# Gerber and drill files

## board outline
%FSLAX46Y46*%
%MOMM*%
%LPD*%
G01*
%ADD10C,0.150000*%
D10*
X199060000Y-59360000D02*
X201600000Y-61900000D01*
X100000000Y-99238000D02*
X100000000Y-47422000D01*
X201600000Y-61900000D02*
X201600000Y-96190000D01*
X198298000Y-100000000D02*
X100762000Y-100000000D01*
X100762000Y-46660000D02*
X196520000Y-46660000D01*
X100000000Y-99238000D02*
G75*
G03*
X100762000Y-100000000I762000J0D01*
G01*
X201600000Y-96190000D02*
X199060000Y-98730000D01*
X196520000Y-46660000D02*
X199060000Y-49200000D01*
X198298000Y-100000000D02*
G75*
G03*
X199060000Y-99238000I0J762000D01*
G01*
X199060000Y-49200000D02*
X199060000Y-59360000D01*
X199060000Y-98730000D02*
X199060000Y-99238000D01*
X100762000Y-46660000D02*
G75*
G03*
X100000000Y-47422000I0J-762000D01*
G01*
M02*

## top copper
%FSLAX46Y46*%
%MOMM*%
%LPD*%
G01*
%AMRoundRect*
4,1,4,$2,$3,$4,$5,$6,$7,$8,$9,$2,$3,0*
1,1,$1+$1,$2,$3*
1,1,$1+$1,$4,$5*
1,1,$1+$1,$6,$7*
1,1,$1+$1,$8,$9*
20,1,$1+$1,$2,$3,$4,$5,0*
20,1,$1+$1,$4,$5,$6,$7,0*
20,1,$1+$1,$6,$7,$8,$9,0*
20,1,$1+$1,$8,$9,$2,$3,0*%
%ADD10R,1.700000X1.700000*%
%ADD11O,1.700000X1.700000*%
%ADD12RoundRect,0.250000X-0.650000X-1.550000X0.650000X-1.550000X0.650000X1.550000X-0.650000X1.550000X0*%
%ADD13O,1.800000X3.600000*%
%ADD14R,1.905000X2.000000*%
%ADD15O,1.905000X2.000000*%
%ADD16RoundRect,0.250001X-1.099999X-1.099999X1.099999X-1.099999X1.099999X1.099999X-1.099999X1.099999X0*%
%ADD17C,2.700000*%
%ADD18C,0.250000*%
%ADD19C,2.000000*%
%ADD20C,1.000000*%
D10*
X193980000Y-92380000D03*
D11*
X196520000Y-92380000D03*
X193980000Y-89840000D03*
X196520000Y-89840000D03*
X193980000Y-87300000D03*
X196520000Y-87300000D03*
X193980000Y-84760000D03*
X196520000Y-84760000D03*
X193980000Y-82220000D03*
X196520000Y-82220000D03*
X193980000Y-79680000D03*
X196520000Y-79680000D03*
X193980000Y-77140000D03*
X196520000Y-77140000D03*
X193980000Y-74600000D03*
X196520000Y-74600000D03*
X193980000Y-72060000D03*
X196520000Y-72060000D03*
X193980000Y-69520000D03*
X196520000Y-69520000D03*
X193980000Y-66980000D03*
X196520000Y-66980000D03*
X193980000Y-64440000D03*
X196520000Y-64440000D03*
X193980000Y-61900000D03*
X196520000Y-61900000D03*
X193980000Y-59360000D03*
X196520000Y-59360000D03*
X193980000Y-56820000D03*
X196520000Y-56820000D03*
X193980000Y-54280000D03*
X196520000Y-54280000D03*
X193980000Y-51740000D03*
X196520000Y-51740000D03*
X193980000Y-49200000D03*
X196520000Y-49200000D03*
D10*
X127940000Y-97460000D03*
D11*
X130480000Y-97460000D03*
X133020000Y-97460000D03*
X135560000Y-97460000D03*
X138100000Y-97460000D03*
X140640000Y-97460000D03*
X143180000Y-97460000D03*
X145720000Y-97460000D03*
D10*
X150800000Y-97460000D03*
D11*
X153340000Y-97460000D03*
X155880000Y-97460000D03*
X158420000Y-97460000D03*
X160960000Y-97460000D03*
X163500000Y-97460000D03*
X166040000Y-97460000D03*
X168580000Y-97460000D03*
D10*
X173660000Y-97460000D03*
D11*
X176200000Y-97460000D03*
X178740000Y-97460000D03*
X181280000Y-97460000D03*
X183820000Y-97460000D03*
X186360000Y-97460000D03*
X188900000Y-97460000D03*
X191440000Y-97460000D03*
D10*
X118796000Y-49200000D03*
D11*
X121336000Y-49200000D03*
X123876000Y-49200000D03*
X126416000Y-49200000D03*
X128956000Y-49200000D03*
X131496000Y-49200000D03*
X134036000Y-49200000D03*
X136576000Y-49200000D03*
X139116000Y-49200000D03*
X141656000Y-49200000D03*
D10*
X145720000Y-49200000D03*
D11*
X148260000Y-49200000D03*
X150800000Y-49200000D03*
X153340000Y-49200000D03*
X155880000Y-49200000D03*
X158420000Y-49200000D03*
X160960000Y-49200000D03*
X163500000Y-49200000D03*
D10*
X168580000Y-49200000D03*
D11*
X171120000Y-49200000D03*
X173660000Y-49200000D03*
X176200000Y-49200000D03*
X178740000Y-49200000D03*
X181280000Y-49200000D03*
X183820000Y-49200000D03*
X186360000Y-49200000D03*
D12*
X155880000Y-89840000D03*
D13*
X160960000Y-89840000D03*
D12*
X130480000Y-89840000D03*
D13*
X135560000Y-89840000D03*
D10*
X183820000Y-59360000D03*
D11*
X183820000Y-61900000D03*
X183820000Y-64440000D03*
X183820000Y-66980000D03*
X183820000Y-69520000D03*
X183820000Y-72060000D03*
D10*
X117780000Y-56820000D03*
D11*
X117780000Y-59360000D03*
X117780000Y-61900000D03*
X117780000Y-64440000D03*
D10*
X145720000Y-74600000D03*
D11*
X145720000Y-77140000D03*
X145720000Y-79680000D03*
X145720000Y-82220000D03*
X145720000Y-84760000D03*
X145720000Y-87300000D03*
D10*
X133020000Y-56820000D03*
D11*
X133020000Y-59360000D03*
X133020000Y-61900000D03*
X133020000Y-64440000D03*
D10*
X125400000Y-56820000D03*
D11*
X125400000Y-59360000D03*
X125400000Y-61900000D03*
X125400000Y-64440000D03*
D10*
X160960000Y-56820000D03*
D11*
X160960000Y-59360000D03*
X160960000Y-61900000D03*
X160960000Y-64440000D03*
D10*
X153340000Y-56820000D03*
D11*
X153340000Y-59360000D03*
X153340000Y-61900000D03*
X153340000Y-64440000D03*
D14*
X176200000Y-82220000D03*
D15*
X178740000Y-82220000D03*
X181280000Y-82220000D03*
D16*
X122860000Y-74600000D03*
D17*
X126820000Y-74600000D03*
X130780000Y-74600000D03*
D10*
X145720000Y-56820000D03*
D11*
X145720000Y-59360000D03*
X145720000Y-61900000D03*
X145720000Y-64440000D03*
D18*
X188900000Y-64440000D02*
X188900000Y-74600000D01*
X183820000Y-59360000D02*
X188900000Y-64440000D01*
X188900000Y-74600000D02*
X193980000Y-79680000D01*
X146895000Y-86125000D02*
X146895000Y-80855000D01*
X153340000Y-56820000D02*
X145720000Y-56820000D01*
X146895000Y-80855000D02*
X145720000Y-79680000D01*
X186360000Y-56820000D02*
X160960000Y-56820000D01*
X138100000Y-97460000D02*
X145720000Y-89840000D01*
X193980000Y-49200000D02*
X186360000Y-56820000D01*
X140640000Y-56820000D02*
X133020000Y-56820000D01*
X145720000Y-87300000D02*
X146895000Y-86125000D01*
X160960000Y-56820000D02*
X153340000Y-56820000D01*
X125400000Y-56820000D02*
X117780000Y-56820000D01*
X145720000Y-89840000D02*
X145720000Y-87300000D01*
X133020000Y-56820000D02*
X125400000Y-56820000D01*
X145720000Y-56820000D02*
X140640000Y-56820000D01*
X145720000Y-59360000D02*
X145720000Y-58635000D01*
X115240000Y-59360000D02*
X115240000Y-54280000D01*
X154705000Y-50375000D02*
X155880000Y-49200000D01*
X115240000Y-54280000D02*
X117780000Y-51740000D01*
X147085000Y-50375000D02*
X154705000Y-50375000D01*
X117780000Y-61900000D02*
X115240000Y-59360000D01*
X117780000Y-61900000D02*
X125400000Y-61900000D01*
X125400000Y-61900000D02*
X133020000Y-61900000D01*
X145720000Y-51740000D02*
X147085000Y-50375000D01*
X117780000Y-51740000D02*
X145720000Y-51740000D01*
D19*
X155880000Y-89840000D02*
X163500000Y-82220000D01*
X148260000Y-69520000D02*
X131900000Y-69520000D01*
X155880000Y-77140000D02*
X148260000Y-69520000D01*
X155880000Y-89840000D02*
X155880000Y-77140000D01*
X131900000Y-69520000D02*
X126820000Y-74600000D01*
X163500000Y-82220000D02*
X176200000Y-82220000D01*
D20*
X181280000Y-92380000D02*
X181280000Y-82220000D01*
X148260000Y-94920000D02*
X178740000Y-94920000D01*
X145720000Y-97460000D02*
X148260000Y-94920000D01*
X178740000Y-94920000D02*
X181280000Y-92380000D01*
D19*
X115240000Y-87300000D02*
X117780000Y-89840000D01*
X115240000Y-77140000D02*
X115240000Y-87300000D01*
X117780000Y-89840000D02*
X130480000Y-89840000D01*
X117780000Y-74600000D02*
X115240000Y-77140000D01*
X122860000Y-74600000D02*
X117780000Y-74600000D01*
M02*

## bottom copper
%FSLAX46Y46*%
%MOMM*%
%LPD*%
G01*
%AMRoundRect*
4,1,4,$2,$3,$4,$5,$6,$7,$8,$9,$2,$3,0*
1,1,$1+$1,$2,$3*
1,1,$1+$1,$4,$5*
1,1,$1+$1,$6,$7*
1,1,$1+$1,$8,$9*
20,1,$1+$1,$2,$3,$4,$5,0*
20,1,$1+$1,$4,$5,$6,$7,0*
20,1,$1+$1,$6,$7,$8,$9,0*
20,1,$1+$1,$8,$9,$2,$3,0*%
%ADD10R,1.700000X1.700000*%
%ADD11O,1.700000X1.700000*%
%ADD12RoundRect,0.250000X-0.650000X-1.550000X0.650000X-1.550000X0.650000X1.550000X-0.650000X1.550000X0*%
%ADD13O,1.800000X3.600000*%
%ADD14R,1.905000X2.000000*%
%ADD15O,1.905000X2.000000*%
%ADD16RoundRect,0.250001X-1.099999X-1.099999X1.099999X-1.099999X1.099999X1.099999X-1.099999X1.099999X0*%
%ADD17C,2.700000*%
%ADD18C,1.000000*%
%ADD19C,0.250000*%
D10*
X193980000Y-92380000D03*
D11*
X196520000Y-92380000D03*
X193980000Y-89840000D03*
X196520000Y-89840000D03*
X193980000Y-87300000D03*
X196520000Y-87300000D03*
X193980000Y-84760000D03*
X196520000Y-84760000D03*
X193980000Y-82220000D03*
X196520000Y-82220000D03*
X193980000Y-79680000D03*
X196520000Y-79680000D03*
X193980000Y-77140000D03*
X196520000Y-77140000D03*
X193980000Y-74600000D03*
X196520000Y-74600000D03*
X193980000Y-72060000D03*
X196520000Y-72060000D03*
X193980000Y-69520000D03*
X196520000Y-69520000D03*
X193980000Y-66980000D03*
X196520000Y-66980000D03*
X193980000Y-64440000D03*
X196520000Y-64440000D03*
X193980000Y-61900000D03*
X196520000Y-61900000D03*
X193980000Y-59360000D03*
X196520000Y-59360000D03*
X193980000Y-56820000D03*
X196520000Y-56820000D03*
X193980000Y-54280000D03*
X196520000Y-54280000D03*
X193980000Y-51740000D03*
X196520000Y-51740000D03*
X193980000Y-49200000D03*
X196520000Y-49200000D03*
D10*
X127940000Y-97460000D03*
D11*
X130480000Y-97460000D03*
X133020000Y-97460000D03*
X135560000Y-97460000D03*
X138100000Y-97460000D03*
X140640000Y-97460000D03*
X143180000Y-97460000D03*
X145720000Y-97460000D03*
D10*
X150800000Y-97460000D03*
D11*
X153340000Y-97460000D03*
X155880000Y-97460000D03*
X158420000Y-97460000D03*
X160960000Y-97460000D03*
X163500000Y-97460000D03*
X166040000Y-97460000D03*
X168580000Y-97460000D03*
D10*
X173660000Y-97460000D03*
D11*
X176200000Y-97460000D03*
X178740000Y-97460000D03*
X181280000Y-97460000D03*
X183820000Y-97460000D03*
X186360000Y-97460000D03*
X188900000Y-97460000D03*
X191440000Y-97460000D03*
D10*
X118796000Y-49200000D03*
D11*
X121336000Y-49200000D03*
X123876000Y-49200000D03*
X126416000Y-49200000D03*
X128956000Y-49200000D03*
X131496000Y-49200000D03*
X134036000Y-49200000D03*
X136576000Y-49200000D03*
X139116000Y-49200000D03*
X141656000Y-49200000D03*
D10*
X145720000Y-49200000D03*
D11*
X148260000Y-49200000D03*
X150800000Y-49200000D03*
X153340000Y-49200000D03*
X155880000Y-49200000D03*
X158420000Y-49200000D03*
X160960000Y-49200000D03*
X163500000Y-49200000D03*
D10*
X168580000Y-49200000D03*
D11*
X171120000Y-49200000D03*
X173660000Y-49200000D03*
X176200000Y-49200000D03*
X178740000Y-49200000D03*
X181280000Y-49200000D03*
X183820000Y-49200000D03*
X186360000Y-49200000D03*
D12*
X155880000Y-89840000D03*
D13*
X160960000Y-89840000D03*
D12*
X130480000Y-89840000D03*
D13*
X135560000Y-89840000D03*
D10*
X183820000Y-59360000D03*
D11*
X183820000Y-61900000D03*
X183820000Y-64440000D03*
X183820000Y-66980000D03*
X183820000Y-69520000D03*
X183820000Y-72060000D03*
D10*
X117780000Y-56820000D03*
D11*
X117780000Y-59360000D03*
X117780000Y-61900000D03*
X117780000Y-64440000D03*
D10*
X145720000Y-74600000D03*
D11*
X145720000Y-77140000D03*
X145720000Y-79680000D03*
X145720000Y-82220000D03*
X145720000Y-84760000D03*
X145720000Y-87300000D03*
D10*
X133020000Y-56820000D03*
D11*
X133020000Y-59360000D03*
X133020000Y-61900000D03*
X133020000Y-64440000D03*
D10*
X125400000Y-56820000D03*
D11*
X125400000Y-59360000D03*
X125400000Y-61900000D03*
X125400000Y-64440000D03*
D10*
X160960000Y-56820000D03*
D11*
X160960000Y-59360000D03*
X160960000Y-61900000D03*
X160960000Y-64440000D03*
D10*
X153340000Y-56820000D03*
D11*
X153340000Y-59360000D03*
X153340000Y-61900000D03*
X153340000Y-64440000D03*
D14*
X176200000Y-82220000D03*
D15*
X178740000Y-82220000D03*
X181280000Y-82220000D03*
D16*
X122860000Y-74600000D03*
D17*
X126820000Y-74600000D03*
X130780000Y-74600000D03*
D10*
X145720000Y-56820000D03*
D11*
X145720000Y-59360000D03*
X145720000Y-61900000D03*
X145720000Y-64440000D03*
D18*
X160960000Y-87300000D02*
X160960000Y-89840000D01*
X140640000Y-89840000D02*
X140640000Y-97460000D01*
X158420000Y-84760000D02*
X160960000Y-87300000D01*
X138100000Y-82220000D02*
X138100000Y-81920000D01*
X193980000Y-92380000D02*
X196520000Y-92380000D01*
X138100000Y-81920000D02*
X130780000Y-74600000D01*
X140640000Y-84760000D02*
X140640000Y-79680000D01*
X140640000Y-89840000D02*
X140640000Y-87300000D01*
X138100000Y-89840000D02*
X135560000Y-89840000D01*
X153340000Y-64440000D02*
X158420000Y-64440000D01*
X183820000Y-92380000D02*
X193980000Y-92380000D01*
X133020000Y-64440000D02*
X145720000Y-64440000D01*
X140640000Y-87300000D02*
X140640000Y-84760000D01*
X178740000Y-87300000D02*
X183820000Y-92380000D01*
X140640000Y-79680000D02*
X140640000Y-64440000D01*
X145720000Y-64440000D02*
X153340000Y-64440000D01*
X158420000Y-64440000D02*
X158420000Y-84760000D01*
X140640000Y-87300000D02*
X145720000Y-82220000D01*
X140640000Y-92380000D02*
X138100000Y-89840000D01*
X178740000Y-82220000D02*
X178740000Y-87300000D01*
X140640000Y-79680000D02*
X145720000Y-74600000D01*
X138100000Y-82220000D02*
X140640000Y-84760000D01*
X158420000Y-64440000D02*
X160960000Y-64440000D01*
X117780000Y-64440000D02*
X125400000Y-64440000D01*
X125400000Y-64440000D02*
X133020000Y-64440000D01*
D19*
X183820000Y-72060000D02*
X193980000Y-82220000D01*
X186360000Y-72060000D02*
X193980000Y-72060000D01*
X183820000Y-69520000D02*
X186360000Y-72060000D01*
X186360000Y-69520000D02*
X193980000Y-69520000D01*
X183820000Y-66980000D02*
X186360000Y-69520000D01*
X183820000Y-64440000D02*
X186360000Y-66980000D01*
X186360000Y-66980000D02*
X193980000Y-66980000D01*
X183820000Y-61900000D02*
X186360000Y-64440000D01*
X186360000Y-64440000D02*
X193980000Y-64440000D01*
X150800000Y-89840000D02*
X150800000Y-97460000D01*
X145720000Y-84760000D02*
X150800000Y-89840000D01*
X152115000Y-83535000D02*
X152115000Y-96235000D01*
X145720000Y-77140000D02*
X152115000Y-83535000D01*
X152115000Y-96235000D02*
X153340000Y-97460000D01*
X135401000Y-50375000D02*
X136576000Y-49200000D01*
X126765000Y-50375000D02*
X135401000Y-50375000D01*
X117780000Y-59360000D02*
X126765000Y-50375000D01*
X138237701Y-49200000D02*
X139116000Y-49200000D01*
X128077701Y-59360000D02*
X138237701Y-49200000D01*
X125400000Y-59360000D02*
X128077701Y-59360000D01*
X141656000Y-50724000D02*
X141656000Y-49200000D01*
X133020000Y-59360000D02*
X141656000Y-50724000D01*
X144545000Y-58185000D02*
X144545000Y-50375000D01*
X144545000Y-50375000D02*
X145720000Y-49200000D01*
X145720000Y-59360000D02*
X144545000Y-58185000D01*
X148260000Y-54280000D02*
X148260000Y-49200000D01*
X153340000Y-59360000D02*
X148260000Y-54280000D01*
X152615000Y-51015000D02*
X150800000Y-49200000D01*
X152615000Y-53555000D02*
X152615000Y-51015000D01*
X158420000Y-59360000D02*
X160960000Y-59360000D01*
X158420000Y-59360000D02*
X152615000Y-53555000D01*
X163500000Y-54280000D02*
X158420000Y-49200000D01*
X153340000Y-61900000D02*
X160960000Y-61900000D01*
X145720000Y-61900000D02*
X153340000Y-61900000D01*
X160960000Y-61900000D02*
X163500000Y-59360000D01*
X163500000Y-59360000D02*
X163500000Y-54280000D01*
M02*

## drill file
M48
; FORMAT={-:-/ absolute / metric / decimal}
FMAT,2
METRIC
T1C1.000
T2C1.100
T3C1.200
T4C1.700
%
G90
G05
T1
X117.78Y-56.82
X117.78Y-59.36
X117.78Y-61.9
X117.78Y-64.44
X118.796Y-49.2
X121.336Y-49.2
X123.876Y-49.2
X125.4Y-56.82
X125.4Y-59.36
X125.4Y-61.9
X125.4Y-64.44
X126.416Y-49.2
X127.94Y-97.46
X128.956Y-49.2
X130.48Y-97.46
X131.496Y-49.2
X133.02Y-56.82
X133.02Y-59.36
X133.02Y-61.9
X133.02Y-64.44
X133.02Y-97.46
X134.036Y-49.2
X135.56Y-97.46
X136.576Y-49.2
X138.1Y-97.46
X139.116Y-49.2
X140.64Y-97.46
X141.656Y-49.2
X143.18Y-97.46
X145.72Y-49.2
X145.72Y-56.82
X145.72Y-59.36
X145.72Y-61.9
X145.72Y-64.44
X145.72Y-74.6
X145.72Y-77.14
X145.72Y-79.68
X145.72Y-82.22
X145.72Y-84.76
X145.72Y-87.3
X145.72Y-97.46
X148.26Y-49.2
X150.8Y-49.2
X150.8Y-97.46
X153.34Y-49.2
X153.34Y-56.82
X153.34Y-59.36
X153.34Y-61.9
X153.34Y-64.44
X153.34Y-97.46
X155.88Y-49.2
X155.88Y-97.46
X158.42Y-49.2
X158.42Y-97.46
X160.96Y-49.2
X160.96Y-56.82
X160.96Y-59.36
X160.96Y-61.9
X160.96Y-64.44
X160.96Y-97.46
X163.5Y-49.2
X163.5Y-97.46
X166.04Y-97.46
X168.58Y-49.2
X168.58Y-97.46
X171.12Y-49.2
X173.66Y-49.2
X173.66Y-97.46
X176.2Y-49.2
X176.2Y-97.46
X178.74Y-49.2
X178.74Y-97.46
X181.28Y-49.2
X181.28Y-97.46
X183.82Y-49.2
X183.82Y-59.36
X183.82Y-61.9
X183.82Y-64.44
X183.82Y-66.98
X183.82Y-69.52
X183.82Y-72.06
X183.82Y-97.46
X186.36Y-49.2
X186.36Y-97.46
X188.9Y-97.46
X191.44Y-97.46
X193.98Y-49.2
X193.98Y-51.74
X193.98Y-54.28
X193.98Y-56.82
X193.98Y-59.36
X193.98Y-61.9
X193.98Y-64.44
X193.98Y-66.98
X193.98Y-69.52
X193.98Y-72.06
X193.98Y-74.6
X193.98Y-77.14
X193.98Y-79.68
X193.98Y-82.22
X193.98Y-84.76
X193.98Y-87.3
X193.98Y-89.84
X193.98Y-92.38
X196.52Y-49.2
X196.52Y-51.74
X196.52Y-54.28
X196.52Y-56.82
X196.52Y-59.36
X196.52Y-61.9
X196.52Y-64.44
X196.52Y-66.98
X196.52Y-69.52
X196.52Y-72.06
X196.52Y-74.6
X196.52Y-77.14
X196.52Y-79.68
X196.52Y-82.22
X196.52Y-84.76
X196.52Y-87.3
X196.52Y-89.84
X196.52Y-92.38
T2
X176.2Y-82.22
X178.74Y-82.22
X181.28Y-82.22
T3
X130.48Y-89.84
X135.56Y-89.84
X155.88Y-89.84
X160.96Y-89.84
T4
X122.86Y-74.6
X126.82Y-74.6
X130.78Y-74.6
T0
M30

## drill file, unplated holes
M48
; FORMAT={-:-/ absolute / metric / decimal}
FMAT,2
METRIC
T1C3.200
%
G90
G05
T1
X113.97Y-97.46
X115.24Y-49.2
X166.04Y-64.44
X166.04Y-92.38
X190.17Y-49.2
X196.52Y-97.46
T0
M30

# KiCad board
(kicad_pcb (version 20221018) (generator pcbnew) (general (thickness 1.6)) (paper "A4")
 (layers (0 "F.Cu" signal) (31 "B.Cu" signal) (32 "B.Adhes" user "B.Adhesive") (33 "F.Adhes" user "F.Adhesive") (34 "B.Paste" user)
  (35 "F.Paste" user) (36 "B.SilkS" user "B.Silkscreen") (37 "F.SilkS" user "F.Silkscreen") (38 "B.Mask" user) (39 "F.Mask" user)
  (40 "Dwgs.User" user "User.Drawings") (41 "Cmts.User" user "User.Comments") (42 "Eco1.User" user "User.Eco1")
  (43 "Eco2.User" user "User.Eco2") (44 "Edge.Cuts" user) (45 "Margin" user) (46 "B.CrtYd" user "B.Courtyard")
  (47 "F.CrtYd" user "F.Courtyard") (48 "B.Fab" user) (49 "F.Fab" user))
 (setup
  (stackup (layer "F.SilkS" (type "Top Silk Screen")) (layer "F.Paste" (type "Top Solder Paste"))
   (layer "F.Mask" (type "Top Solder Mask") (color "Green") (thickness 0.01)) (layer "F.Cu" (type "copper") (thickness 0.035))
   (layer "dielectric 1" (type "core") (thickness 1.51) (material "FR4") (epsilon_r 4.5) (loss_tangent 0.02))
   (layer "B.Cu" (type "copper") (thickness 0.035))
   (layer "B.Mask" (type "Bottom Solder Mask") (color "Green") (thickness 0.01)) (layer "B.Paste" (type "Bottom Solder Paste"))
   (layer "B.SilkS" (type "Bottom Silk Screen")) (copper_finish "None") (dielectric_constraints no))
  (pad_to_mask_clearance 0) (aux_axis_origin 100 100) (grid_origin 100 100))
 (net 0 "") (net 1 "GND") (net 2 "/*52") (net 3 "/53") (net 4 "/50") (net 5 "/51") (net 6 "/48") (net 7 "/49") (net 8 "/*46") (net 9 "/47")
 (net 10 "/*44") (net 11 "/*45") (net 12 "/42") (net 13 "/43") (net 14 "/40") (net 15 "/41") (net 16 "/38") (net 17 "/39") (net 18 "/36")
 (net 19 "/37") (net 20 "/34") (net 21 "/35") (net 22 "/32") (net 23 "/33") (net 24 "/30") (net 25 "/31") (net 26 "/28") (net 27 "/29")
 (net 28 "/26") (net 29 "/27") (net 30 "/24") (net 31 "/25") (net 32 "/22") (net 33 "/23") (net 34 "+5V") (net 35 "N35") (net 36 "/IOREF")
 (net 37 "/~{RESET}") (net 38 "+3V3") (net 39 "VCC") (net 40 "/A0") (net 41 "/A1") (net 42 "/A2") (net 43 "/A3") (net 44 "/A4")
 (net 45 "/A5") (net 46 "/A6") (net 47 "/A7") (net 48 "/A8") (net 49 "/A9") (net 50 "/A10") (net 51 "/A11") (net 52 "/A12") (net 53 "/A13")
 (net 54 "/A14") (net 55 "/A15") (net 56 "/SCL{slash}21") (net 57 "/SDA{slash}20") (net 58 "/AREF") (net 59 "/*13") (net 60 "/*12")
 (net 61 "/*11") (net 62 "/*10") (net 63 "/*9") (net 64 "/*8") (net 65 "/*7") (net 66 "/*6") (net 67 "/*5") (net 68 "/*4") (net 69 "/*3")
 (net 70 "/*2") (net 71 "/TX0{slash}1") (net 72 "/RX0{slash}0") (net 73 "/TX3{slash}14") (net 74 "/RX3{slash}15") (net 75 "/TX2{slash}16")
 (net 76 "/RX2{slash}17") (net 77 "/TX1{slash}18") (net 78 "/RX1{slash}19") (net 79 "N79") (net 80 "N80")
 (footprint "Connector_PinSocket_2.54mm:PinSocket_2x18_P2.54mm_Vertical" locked (layer "F.Cu") (at 193.98 92.38 180)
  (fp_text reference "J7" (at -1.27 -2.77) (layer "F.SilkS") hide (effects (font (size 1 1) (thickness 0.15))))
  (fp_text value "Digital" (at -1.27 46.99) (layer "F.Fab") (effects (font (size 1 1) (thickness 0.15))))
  (pad "1" thru_hole rect locked (at 0 0 180) (size 1.7 1.7) (drill 1) (layers "*.Cu" "*.Mask") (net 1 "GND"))
  (pad "2" thru_hole oval locked (at -2.54 0 180) (size 1.7 1.7) (drill 1) (layers "*.Cu" "*.Mask") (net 1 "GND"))
  (pad "3" thru_hole oval locked (at 0 2.54 180) (size 1.7 1.7) (drill 1) (layers "*.Cu" "*.Mask") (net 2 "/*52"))
  (pad "4" thru_hole oval locked (at -2.54 2.54 180) (size 1.7 1.7) (drill 1) (layers "*.Cu" "*.Mask") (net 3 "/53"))
  (pad "5" thru_hole oval locked (at 0 5.08 180) (size 1.7 1.7) (drill 1) (layers "*.Cu" "*.Mask") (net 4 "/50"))
  (pad "6" thru_hole oval locked (at -2.54 5.08 180) (size 1.7 1.7) (drill 1) (layers "*.Cu" "*.Mask") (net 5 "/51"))
  (pad "7" thru_hole oval locked (at 0 7.62 180) (size 1.7 1.7) (drill 1) (layers "*.Cu" "*.Mask") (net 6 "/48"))
  (pad "8" thru_hole oval locked (at -2.54 7.62 180) (size 1.7 1.7) (drill 1) (layers "*.Cu" "*.Mask") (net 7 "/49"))
  (pad "9" thru_hole oval locked (at 0 10.16 180) (size 1.7 1.7) (drill 1) (layers "*.Cu" "*.Mask") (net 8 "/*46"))
  (pad "10" thru_hole oval locked (at -2.54 10.16 180) (size 1.7 1.7) (drill 1) (layers "*.Cu" "*.Mask") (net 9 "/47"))
  (pad "11" thru_hole oval locked (at 0 12.7 180) (size 1.7 1.7) (drill 1) (layers "*.Cu" "*.Mask") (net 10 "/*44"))
  (pad "12" thru_hole oval locked (at -2.54 12.7 180) (size 1.7 1.7) (drill 1) (layers "*.Cu" "*.Mask") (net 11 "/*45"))
  (pad "13" thru_hole oval locked (at 0 15.24 180) (size 1.7 1.7) (drill 1) (layers "*.Cu" "*.Mask") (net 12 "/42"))
  (pad "14" thru_hole oval locked (at -2.54 15.24 180) (size 1.7 1.7) (drill 1) (layers "*.Cu" "*.Mask") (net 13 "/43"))
  (pad "15" thru_hole oval locked (at 0 17.78 180) (size 1.7 1.7) (drill 1) (layers "*.Cu" "*.Mask") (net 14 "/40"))
  (pad "16" thru_hole oval locked (at -2.54 17.78 180) (size 1.7 1.7) (drill 1) (layers "*.Cu" "*.Mask") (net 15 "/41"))
  (pad "17" thru_hole oval locked (at 0 20.32 180) (size 1.7 1.7) (drill 1) (layers "*.Cu" "*.Mask") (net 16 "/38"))
  (pad "18" thru_hole oval locked (at -2.54 20.32 180) (size 1.7 1.7) (drill 1) (layers "*.Cu" "*.Mask") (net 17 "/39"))
  (pad "19" thru_hole oval locked (at 0 22.86 180) (size 1.7 1.7) (drill 1) (layers "*.Cu" "*.Mask") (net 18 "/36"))
  (pad "20" thru_hole oval locked (at -2.54 22.86 180) (size 1.7 1.7) (drill 1) (layers "*.Cu" "*.Mask") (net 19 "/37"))
  (pad "21" thru_hole oval locked (at 0 25.4 180) (size 1.7 1.7) (drill 1) (layers "*.Cu" "*.Mask") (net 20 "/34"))
  (pad "22" thru_hole oval locked (at -2.54 25.4 180) (size 1.7 1.7) (drill 1) (layers "*.Cu" "*.Mask") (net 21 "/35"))
  (pad "23" thru_hole oval locked (at 0 27.94 180) (size 1.7 1.7) (drill 1) (layers "*.Cu" "*.Mask") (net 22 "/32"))
  (pad "24" thru_hole oval locked (at -2.54 27.94 180) (size 1.7 1.7) (drill 1) (layers "*.Cu" "*.Mask") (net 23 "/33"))
  (pad "25" thru_hole oval locked (at 0 30.48 180) (size 1.7 1.7) (drill 1) (layers "*.Cu" "*.Mask") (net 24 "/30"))
  (pad "26" thru_hole oval locked (at -2.54 30.48 180) (size 1.7 1.7) (drill 1) (layers "*.Cu" "*.Mask") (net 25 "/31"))
  (pad "27" thru_hole oval locked (at 0 33.02 180) (size 1.7 1.7) (drill 1) (layers "*.Cu" "*.Mask") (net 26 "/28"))
  (pad "28" thru_hole oval locked (at -2.54 33.02 180) (size 1.7 1.7) (drill 1) (layers "*.Cu" "*.Mask") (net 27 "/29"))
  (pad "29" thru_hole oval locked (at 0 35.56 180) (size 1.7 1.7) (drill 1) (layers "*.Cu" "*.Mask") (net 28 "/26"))
  (pad "30" thru_hole oval locked (at -2.54 35.56 180) (size 1.7 1.7) (drill 1) (layers "*.Cu" "*.Mask") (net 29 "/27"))
  (pad "31" thru_hole oval locked (at 0 38.1 180) (size 1.7 1.7) (drill 1) (layers "*.Cu" "*.Mask") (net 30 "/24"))
  (pad "32" thru_hole oval locked (at -2.54 38.1 180) (size 1.7 1.7) (drill 1) (layers "*.Cu" "*.Mask") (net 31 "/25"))
  (pad "33" thru_hole oval locked (at 0 40.64 180) (size 1.7 1.7) (drill 1) (layers "*.Cu" "*.Mask") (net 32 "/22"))
  (pad "34" thru_hole oval locked (at -2.54 40.64 180) (size 1.7 1.7) (drill 1) (layers "*.Cu" "*.Mask") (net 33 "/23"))
  (pad "35" thru_hole oval locked (at 0 43.18 180) (size 1.7 1.7) (drill 1) (layers "*.Cu" "*.Mask") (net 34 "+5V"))
  (pad "36" thru_hole oval locked (at -2.54 43.18 180) (size 1.7 1.7) (drill 1) (layers "*.Cu" "*.Mask") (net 34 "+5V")))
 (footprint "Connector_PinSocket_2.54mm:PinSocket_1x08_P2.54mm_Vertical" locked (layer "F.Cu") (at 127.94 97.46 90)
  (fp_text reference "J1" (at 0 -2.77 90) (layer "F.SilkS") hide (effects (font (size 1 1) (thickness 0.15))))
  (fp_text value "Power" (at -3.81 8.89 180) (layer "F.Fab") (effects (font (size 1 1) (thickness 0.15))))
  (pad "1" thru_hole rect locked (at 0 0 90) (size 1.7 1.7) (drill 1) (layers "*.Cu" "*.Mask") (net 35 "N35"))
  (pad "2" thru_hole oval locked (at 0 2.54 90) (size 1.7 1.7) (drill 1) (layers "*.Cu" "*.Mask") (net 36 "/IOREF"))
  (pad "3" thru_hole oval locked (at 0 5.08 90) (size 1.7 1.7) (drill 1) (layers "*.Cu" "*.Mask") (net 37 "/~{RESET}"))
  (pad "4" thru_hole oval locked (at 0 7.62 90) (size 1.7 1.7) (drill 1) (layers "*.Cu" "*.Mask") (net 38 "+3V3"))
  (pad "5" thru_hole oval locked (at 0 10.16 90) (size 1.7 1.7) (drill 1) (layers "*.Cu" "*.Mask") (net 34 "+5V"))
  (pad "6" thru_hole oval locked (at 0 12.7 90) (size 1.7 1.7) (drill 1) (layers "*.Cu" "*.Mask") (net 1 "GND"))
  (pad "7" thru_hole oval locked (at 0 15.24 90) (size 1.7 1.7) (drill 1) (layers "*.Cu" "*.Mask") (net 1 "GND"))
  (pad "8" thru_hole oval locked (at 0 17.78 90) (size 1.7 1.7) (drill 1) (layers "*.Cu" "*.Mask") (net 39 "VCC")))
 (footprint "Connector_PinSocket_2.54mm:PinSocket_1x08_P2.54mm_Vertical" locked (layer "F.Cu") (at 150.8 97.46 90)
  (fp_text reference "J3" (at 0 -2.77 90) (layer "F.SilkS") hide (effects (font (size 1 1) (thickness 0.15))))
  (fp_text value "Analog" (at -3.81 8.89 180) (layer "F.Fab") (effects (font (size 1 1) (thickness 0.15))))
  (pad "1" thru_hole rect locked (at 0 0 90) (size 1.7 1.7) (drill 1) (layers "*.Cu" "*.Mask") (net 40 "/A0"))
  (pad "2" thru_hole oval locked (at 0 2.54 90) (size 1.7 1.7) (drill 1) (layers "*.Cu" "*.Mask") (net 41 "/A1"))
  (pad "3" thru_hole oval locked (at 0 5.08 90) (size 1.7 1.7) (drill 1) (layers "*.Cu" "*.Mask") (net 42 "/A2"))
  (pad "4" thru_hole oval locked (at 0 7.62 90) (size 1.7 1.7) (drill 1) (layers "*.Cu" "*.Mask") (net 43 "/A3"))
  (pad "5" thru_hole oval locked (at 0 10.16 90) (size 1.7 1.7) (drill 1) (layers "*.Cu" "*.Mask") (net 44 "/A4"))
  (pad "6" thru_hole oval locked (at 0 12.7 90) (size 1.7 1.7) (drill 1) (layers "*.Cu" "*.Mask") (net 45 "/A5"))
  (pad "7" thru_hole oval locked (at 0 15.24 90) (size 1.7 1.7) (drill 1) (layers "*.Cu" "*.Mask") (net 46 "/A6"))
  (pad "8" thru_hole oval locked (at 0 17.78 90) (size 1.7 1.7) (drill 1) (layers "*.Cu" "*.Mask") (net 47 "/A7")))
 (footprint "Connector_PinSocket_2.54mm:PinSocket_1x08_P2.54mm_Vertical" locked (layer "F.Cu") (at 173.66 97.46 90)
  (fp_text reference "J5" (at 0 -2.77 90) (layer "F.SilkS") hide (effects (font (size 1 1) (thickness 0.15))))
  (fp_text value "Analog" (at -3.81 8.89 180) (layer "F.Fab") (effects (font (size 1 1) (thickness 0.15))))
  (pad "1" thru_hole rect locked (at 0 0 90) (size 1.7 1.7) (drill 1) (layers "*.Cu" "*.Mask") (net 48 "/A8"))
  (pad "2" thru_hole oval locked (at 0 2.54 90) (size 1.7 1.7) (drill 1) (layers "*.Cu" "*.Mask") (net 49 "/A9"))
  (pad "3" thru_hole oval locked (at 0 5.08 90) (size 1.7 1.7) (drill 1) (layers "*.Cu" "*.Mask") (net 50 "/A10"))
  (pad "4" thru_hole oval locked (at 0 7.62 90) (size 1.7 1.7) (drill 1) (layers "*.Cu" "*.Mask") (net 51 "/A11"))
  (pad "5" thru_hole oval locked (at 0 10.16 90) (size 1.7 1.7) (drill 1) (layers "*.Cu" "*.Mask") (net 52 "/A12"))
  (pad "6" thru_hole oval locked (at 0 12.7 90) (size 1.7 1.7) (drill 1) (layers "*.Cu" "*.Mask") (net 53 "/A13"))
  (pad "7" thru_hole oval locked (at 0 15.24 90) (size 1.7 1.7) (drill 1) (layers "*.Cu" "*.Mask") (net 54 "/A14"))
  (pad "8" thru_hole oval locked (at 0 17.78 90) (size 1.7 1.7) (drill 1) (layers "*.Cu" "*.Mask") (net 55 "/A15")))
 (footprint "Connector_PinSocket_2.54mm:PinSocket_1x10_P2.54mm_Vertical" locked (layer "F.Cu") (at 118.796 49.2 90)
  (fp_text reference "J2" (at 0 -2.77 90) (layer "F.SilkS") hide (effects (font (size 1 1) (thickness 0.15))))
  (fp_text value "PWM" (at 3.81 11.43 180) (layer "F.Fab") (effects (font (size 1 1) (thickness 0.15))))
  (pad "1" thru_hole rect locked (at 0 0 90) (size 1.7 1.7) (drill 1) (layers "*.Cu" "*.Mask") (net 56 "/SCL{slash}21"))
  (pad "2" thru_hole oval locked (at 0 2.54 90) (size 1.7 1.7) (drill 1) (layers "*.Cu" "*.Mask") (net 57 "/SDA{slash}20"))
  (pad "3" thru_hole oval locked (at 0 5.08 90) (size 1.7 1.7) (drill 1) (layers "*.Cu" "*.Mask") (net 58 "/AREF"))
  (pad "4" thru_hole oval locked (at 0 7.62 90) (size 1.7 1.7) (drill 1) (layers "*.Cu" "*.Mask") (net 1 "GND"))
  (pad "5" thru_hole oval locked (at 0 10.16 90) (size 1.7 1.7) (drill 1) (layers "*.Cu" "*.Mask") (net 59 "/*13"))
  (pad "6" thru_hole oval locked (at 0 12.7 90) (size 1.7 1.7) (drill 1) (layers "*.Cu" "*.Mask") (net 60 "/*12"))
  (pad "7" thru_hole oval locked (at 0 15.24 90) (size 1.7 1.7) (drill 1) (layers "*.Cu" "*.Mask") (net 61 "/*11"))
  (pad "8" thru_hole oval locked (at 0 17.78 90) (size 1.7 1.7) (drill 1) (layers "*.Cu" "*.Mask") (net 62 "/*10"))
  (pad "9" thru_hole oval locked (at 0 20.32 90) (size 1.7 1.7) (drill 1) (layers "*.Cu" "*.Mask") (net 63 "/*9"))
  (pad "10" thru_hole oval locked (at 0 22.86 90) (size 1.7 1.7) (drill 1) (layers "*.Cu" "*.Mask") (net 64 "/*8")))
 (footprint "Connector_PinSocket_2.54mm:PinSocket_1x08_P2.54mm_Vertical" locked (layer "F.Cu") (at 145.72 49.2 90)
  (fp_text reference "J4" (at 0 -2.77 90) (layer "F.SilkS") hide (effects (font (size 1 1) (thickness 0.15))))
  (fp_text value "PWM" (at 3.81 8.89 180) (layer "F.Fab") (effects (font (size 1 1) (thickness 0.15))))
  (pad "1" thru_hole rect locked (at 0 0 90) (size 1.7 1.7) (drill 1) (layers "*.Cu" "*.Mask") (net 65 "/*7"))
  (pad "2" thru_hole oval locked (at 0 2.54 90) (size 1.7 1.7) (drill 1) (layers "*.Cu" "*.Mask") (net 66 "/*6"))
  (pad "3" thru_hole oval locked (at 0 5.08 90) (size 1.7 1.7) (drill 1) (layers "*.Cu" "*.Mask") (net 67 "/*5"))
  (pad "4" thru_hole oval locked (at 0 7.62 90) (size 1.7 1.7) (drill 1) (layers "*.Cu" "*.Mask") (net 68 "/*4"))
  (pad "5" thru_hole oval locked (at 0 10.16 90) (size 1.7 1.7) (drill 1) (layers "*.Cu" "*.Mask") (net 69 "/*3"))
  (pad "6" thru_hole oval locked (at 0 12.7 90) (size 1.7 1.7) (drill 1) (layers "*.Cu" "*.Mask") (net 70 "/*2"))
  (pad "7" thru_hole oval locked (at 0 15.24 90) (size 1.7 1.7) (drill 1) (layers "*.Cu" "*.Mask") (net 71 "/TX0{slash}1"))
  (pad "8" thru_hole oval locked (at 0 17.78 90) (size 1.7 1.7) (drill 1) (layers "*.Cu" "*.Mask") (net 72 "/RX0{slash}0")))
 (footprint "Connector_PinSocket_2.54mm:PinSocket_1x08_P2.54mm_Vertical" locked (layer "F.Cu") (at 168.58 49.2 90)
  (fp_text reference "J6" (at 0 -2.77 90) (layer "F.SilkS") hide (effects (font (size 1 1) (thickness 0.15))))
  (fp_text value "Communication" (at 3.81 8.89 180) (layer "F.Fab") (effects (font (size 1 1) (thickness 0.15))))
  (pad "1" thru_hole rect locked (at 0 0 90) (size 1.7 1.7) (drill 1) (layers "*.Cu" "*.Mask") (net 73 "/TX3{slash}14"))
  (pad "2" thru_hole oval locked (at 0 2.54 90) (size 1.7 1.7) (drill 1) (layers "*.Cu" "*.Mask") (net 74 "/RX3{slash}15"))
  (pad "3" thru_hole oval locked (at 0 5.08 90) (size 1.7 1.7) (drill 1) (layers "*.Cu" "*.Mask") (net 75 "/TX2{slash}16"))
  (pad "4" thru_hole oval locked (at 0 7.62 90) (size 1.7 1.7) (drill 1) (layers "*.Cu" "*.Mask") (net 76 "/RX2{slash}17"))
  (pad "5" thru_hole oval locked (at 0 10.16 90) (size 1.7 1.7) (drill 1) (layers "*.Cu" "*.Mask") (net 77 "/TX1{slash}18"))
  (pad "6" thru_hole oval locked (at 0 12.7 90) (size 1.7 1.7) (drill 1) (layers "*.Cu" "*.Mask") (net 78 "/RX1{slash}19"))
  (pad "7" thru_hole oval locked (at 0 15.24 90) (size 1.7 1.7) (drill 1) (layers "*.Cu" "*.Mask") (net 57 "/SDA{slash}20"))
  (pad "8" thru_hole oval locked (at 0 17.78 90) (size 1.7 1.7) (drill 1) (layers "*.Cu" "*.Mask") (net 56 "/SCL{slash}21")))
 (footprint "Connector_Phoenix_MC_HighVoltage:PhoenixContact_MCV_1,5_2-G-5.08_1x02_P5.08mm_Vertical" (layer "F.Cu") (at 155.88 89.84)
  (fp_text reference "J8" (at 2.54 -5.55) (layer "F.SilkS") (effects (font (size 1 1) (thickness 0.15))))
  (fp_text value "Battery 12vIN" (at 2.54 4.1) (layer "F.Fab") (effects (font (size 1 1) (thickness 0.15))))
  (pad "1" thru_hole roundrect (at 0 0) (size 1.8 3.6) (drill 1.2) (layers "*.Cu" "*.Mask") (roundrect_rratio 0.1388888889) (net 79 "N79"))
  (pad "2" thru_hole oval (at 5.08 0) (size 1.8 3.6) (drill 1.2) (layers "*.Cu" "*.Mask") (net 1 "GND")))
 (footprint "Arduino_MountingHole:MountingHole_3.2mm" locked (layer "F.Cu") (at 196.52 97.46)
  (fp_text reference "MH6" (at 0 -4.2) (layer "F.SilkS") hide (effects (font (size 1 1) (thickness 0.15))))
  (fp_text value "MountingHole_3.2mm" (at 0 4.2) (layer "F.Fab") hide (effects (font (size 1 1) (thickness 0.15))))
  (pad "" np_thru_hole circle locked (at 0 0) (size 3.2 3.2) (drill 3.2) (layers "*.Cu" "*.Mask")))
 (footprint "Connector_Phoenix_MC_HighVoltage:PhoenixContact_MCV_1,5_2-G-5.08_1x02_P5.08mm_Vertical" (layer "F.Cu") (at 130.48 89.84)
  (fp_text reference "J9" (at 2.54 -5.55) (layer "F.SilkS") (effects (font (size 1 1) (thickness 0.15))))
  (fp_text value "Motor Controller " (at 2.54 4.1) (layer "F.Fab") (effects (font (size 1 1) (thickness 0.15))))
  (pad "1" thru_hole roundrect (at 0 0) (size 1.8 3.6) (drill 1.2) (layers "*.Cu" "*.Mask") (roundrect_rratio 0.1388888889) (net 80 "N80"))
  (pad "2" thru_hole oval (at 5.08 0) (size 1.8 3.6) (drill 1.2) (layers "*.Cu" "*.Mask") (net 1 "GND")))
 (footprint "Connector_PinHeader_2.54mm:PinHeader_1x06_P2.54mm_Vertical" (layer "F.Cu") (at 183.82 59.36)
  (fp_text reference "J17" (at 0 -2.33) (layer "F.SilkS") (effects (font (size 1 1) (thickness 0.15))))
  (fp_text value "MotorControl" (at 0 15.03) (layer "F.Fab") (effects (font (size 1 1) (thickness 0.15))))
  (pad "1" thru_hole rect (at 0 0) (size 1.7 1.7) (drill 1) (layers "*.Cu" "*.Mask") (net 10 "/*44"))
  (pad "2" thru_hole oval (at 0 2.54) (size 1.7 1.7) (drill 1) (layers "*.Cu" "*.Mask") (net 22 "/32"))
  (pad "3" thru_hole oval (at 0 5.08) (size 1.7 1.7) (drill 1) (layers "*.Cu" "*.Mask") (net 20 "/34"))
  (pad "4" thru_hole oval (at 0 7.62) (size 1.7 1.7) (drill 1) (layers "*.Cu" "*.Mask") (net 18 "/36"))
  (pad "5" thru_hole oval (at 0 10.16) (size 1.7 1.7) (drill 1) (layers "*.Cu" "*.Mask") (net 16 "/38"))
  (pad "6" thru_hole oval (at 0 12.7) (size 1.7 1.7) (drill 1) (layers "*.Cu" "*.Mask") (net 8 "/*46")))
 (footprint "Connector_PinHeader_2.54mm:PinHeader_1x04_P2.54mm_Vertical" (layer "F.Cu") (at 117.78 56.82)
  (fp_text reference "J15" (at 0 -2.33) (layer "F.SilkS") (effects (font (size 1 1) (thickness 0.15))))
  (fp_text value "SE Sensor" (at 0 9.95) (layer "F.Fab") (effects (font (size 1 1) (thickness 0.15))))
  (pad "1" thru_hole rect (at 0 0) (size 1.7 1.7) (drill 1) (layers "*.Cu" "*.Mask") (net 34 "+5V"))
  (pad "2" thru_hole oval (at 0 2.54) (size 1.7 1.7) (drill 1) (layers "*.Cu" "*.Mask") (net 62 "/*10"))
  (pad "3" thru_hole oval (at 0 5.08) (size 1.7 1.7) (drill 1) (layers "*.Cu" "*.Mask") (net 69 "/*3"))
  (pad "4" thru_hole oval (at 0 7.62) (size 1.7 1.7) (drill 1) (layers "*.Cu" "*.Mask") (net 1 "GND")))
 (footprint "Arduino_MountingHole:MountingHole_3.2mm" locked (layer "F.Cu") (at 115.24 49.2)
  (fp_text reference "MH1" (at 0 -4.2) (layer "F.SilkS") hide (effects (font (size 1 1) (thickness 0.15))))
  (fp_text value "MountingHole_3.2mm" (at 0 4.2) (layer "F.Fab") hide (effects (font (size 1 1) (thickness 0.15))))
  (pad "" np_thru_hole circle locked (at 0 0) (size 3.2 3.2) (drill 3.2) (layers "*.Cu" "*.Mask")))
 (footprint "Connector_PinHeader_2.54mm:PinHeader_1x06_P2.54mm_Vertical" (layer "F.Cu") (at 145.72 74.6)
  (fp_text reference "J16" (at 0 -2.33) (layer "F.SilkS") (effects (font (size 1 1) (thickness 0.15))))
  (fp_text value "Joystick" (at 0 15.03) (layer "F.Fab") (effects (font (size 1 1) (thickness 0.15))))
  (pad "1" thru_hole rect (at 0 0) (size 1.7 1.7) (drill 1) (layers "*.Cu" "*.Mask") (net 1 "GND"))
  (pad "2" thru_hole oval (at 0 2.54) (size 1.7 1.7) (drill 1) (layers "*.Cu" "*.Mask") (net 41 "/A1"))
  (pad "3" thru_hole oval (at 0 5.08) (size 1.7 1.7) (drill 1) (layers "*.Cu" "*.Mask") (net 34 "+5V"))
  (pad "4" thru_hole oval (at 0 7.62) (size 1.7 1.7) (drill 1) (layers "*.Cu" "*.Mask") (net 1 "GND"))
  (pad "5" thru_hole oval (at 0 10.16) (size 1.7 1.7) (drill 1) (layers "*.Cu" "*.Mask") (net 40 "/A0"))
  (pad "6" thru_hole oval (at 0 12.7) (size 1.7 1.7) (drill 1) (layers "*.Cu" "*.Mask") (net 34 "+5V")))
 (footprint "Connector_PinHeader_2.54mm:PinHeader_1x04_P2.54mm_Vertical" (layer "F.Cu") (at 133.02 56.82)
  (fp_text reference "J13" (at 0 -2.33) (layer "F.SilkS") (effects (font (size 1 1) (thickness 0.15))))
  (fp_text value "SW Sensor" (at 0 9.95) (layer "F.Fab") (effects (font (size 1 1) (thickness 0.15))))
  (pad "1" thru_hole rect (at 0 0) (size 1.7 1.7) (drill 1) (layers "*.Cu" "*.Mask") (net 34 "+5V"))
  (pad "2" thru_hole oval (at 0 2.54) (size 1.7 1.7) (drill 1) (layers "*.Cu" "*.Mask") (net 64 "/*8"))
  (pad "3" thru_hole oval (at 0 5.08) (size 1.7 1.7) (drill 1) (layers "*.Cu" "*.Mask") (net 69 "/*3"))
  (pad "4" thru_hole oval (at 0 7.62) (size 1.7 1.7) (drill 1) (layers "*.Cu" "*.Mask") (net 1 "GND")))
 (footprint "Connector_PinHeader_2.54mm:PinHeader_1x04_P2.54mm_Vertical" (layer "F.Cu") (at 125.4 56.82)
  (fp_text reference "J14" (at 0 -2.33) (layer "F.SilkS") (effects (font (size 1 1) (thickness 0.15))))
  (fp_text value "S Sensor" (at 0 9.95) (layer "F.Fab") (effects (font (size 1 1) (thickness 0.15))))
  (pad "1" thru_hole rect (at 0 0) (size 1.7 1.7) (drill 1) (layers "*.Cu" "*.Mask") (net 34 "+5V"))
  (pad "2" thru_hole oval (at 0 2.54) (size 1.7 1.7) (drill 1) (layers "*.Cu" "*.Mask") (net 63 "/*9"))
  (pad "3" thru_hole oval (at 0 5.08) (size 1.7 1.7) (drill 1) (layers "*.Cu" "*.Mask") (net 69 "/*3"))
  (pad "4" thru_hole oval (at 0 7.62) (size 1.7 1.7) (drill 1) (layers "*.Cu" "*.Mask") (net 1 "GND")))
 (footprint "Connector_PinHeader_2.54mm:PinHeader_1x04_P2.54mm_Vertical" (layer "F.Cu") (at 160.96 56.82)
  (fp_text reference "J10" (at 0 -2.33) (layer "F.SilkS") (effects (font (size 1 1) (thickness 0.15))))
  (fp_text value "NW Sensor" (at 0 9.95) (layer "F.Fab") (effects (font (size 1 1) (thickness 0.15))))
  (pad "1" thru_hole rect (at 0 0) (size 1.7 1.7) (drill 1) (layers "*.Cu" "*.Mask") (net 34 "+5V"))
  (pad "2" thru_hole oval (at 0 2.54) (size 1.7 1.7) (drill 1) (layers "*.Cu" "*.Mask") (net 67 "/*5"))
  (pad "3" thru_hole oval (at 0 5.08) (size 1.7 1.7) (drill 1) (layers "*.Cu" "*.Mask") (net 70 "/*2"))
  (pad "4" thru_hole oval (at 0 7.62) (size 1.7 1.7) (drill 1) (layers "*.Cu" "*.Mask") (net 1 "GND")))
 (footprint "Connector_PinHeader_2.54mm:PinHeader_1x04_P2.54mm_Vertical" (layer "F.Cu") (at 153.34 56.82)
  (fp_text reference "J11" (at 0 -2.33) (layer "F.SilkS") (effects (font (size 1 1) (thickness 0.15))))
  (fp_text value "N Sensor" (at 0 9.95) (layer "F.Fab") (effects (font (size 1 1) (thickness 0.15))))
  (pad "1" thru_hole rect (at 0 0) (size 1.7 1.7) (drill 1) (layers "*.Cu" "*.Mask") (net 34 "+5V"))
  (pad "2" thru_hole oval (at 0 2.54) (size 1.7 1.7) (drill 1) (layers "*.Cu" "*.Mask") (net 66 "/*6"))
  (pad "3" thru_hole oval (at 0 5.08) (size 1.7 1.7) (drill 1) (layers "*.Cu" "*.Mask") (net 70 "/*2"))
  (pad "4" thru_hole oval (at 0 7.62) (size 1.7 1.7) (drill 1) (layers "*.Cu" "*.Mask") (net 1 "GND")))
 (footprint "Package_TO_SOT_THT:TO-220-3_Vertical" (layer "F.Cu") (at 176.2 82.22)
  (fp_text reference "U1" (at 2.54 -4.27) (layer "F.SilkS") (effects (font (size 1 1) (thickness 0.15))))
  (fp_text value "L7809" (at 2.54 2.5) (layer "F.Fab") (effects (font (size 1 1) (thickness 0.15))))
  (pad "1" thru_hole rect (at 0 0) (size 1.905 2) (drill 1.1) (layers "*.Cu" "*.Mask") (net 79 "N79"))
  (pad "2" thru_hole oval (at 2.54 0) (size 1.905 2) (drill 1.1) (layers "*.Cu" "*.Mask") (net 1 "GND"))
  (pad "3" thru_hole oval (at 5.08 0) (size 1.905 2) (drill 1.1) (layers "*.Cu" "*.Mask") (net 39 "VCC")))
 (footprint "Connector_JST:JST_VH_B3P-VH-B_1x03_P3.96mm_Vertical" (layer "F.Cu") (at 122.86 74.6)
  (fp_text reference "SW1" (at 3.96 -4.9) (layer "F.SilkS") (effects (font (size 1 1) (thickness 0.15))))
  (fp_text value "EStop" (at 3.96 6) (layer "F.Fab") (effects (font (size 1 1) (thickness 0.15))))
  (pad "1" thru_hole roundrect (at 0 0) (size 2.7 2.7) (drill 1.7) (layers "*.Cu" "*.Mask") (roundrect_rratio 0.09259296296) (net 80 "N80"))
  (pad "2" thru_hole circle (at 3.96 0) (size 2.7 2.7) (drill 1.7) (layers "*.Cu" "*.Mask") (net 79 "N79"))
  (pad "3" thru_hole circle (at 7.92 0) (size 2.7 2.7) (drill 1.7) (layers "*.Cu" "*.Mask") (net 1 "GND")))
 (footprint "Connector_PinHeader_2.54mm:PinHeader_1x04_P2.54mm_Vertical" (layer "F.Cu") (at 145.72 56.82)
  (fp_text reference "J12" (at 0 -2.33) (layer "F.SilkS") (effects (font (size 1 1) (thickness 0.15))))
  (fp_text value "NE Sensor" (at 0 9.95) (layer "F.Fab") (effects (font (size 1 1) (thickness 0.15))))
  (pad "1" thru_hole rect (at 0 0) (size 1.7 1.7) (drill 1) (layers "*.Cu" "*.Mask") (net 34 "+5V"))
  (pad "2" thru_hole oval (at 0 2.54) (size 1.7 1.7) (drill 1) (layers "*.Cu" "*.Mask") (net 65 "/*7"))
  (pad "3" thru_hole oval (at 0 5.08) (size 1.7 1.7) (drill 1) (layers "*.Cu" "*.Mask") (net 70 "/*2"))
  (pad "4" thru_hole oval (at 0 7.62) (size 1.7 1.7) (drill 1) (layers "*.Cu" "*.Mask") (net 1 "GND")))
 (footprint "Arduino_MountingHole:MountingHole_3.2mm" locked (layer "F.Cu") (at 113.97 97.46)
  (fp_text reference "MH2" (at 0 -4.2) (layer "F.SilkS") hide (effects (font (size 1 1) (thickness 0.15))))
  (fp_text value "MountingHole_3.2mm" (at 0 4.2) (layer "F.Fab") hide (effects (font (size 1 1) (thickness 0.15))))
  (pad "" np_thru_hole circle locked (at 0 0) (size 3.2 3.2) (drill 3.2) (layers "*.Cu" "*.Mask")))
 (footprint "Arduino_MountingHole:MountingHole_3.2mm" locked (layer "F.Cu") (at 166.04 64.44)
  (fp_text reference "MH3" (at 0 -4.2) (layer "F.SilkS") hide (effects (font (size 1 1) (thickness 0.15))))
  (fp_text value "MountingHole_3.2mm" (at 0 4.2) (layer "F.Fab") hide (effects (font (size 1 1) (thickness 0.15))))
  (pad "" np_thru_hole circle locked (at 0 0) (size 3.2 3.2) (drill 3.2) (layers "*.Cu" "*.Mask")))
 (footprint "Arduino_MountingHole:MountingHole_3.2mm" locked (layer "F.Cu") (at 166.04 92.38)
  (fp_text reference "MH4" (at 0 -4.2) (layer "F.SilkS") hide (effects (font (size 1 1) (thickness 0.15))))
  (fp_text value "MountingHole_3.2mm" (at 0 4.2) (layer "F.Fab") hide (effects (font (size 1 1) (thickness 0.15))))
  (pad "" np_thru_hole circle locked (at 0 0) (size 3.2 3.2) (drill 3.2) (layers "*.Cu" "*.Mask")))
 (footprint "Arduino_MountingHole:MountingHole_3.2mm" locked (layer "F.Cu") (at 190.17 49.2)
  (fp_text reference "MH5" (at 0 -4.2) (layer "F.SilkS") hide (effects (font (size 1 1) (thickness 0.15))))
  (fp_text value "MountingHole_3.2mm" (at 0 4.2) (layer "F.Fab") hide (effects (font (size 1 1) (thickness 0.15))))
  (pad "" np_thru_hole circle locked (at 0 0) (size 3.2 3.2) (drill 3.2) (layers "*.Cu" "*.Mask")))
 (gr_line (start 199.06 59.36) (end 201.6 61.9) (stroke (width 0.15) (type solid)) (layer "Edge.Cuts"))
 (gr_line (start 100 99.238) (end 100 47.422) (stroke (width 0.15) (type solid)) (layer "Edge.Cuts"))
 (gr_line (start 201.6 61.9) (end 201.6 96.19) (stroke (width 0.15) (type solid)) (layer "Edge.Cuts"))
 (gr_line (start 198.298 100) (end 100.762 100) (stroke (width 0.15) (type solid)) (layer "Edge.Cuts"))
 (gr_line (start 100.762 46.66) (end 196.52 46.66) (stroke (width 0.15) (type solid)) (layer "Edge.Cuts"))
 (gr_arc (start 100.762 100) (mid 100.223185 99.776815) (end 100 99.238) (stroke (width 0.15) (type solid)) (layer "Edge.Cuts"))
 (gr_line (start 201.6 96.19) (end 199.06 98.73) (stroke (width 0.15) (type solid)) (layer "Edge.Cuts"))
 (gr_line (start 196.52 46.66) (end 199.06 49.2) (stroke (width 0.15) (type solid)) (layer "Edge.Cuts"))
 (gr_arc (start 199.06 99.238) (mid 198.836815 99.776815) (end 198.298 100) (stroke (width 0.15) (type solid)) (layer "Edge.Cuts"))
 (gr_line (start 199.06 49.2) (end 199.06 59.36) (stroke (width 0.15) (type solid)) (layer "Edge.Cuts"))
 (gr_line (start 199.06 98.73) (end 199.06 99.238) (stroke (width 0.15) (type solid)) (layer "Edge.Cuts"))
 (gr_arc (start 100 47.422) (mid 100.223185 46.883185) (end 100.762 46.66) (stroke (width 0.15) (type solid)) (layer "Edge.Cuts"))
 (segment (start 160.96 87.3) (end 160.96 89.84) (width 1) (layer "B.Cu") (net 1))
 (segment (start 140.64 89.84) (end 140.64 97.46) (width 1) (layer "B.Cu") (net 1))
 (segment (start 158.42 84.76) (end 160.96 87.3) (width 1) (layer "B.Cu") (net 1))
 (segment (start 138.1 82.22) (end 138.1 81.92) (width 1) (layer "B.Cu") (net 1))
 (segment (start 193.98 92.38) (end 196.52 92.38) (width 1) (layer "B.Cu") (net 1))
 (segment (start 138.1 81.92) (end 130.78 74.6) (width 1) (layer "B.Cu") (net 1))
 (segment (start 140.64 84.76) (end 140.64 79.68) (width 1) (layer "B.Cu") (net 1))
 (segment (start 140.64 89.84) (end 140.64 87.3) (width 1) (layer "B.Cu") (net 1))
 (segment (start 138.1 89.84) (end 135.56 89.84) (width 1) (layer "B.Cu") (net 1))
 (segment (start 153.34 64.44) (end 158.42 64.44) (width 1) (layer "B.Cu") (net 1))
 (segment (start 183.82 92.38) (end 193.98 92.38) (width 1) (layer "B.Cu") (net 1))
 (segment (start 133.02 64.44) (end 145.72 64.44) (width 1) (layer "B.Cu") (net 1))
 (segment (start 140.64 87.3) (end 140.64 84.76) (width 1) (layer "B.Cu") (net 1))
 (segment (start 178.74 87.3) (end 183.82 92.38) (width 1) (layer "B.Cu") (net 1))
 (segment (start 140.64 79.68) (end 140.64 64.44) (width 1) (layer "B.Cu") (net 1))
 (segment (start 145.72 64.44) (end 153.34 64.44) (width 1) (layer "B.Cu") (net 1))
 (segment (start 158.42 64.44) (end 158.42 84.76) (width 1) (layer "B.Cu") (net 1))
 (segment (start 140.64 87.3) (end 145.72 82.22) (width 1) (layer "B.Cu") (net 1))
 (segment (start 140.64 92.38) (end 138.1 89.84) (width 1) (layer "B.Cu") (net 1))
 (segment (start 178.74 82.22) (end 178.74 87.3) (width 1) (layer "B.Cu") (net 1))
 (segment (start 140.64 79.68) (end 145.72 74.6) (width 1) (layer "B.Cu") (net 1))
 (segment (start 138.1 82.22) (end 140.64 84.76) (width 1) (layer "B.Cu") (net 1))
 (segment (start 158.42 64.44) (end 160.96 64.44) (width 1) (layer "B.Cu") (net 1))
 (segment (start 117.78 64.44) (end 125.4 64.44) (width 1) (layer "B.Cu") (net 1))
 (segment (start 125.4 64.44) (end 133.02 64.44) (width 1) (layer "B.Cu") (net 1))
 (segment (start 183.82 72.06) (end 193.98 82.22) (width 0.25) (layer "B.Cu") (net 8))
 (segment (start 188.9 64.44) (end 188.9 74.6) (width 0.25) (layer "F.Cu") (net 10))
 (segment (start 183.82 59.36) (end 188.9 64.44) (width 0.25) (layer "F.Cu") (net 10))
 (segment (start 188.9 74.6) (end 193.98 79.68) (width 0.25) (layer "F.Cu") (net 10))
 (segment (start 186.36 72.06) (end 193.98 72.06) (width 0.25) (layer "B.Cu") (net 16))
 (segment (start 183.82 69.52) (end 186.36 72.06) (width 0.25) (layer "B.Cu") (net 16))
 (segment (start 186.36 69.52) (end 193.98 69.52) (width 0.25) (layer "B.Cu") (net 18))
 (segment (start 183.82 66.98) (end 186.36 69.52) (width 0.25) (layer "B.Cu") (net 18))
 (segment (start 183.82 64.44) (end 186.36 66.98) (width 0.25) (layer "B.Cu") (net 20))
 (segment (start 186.36 66.98) (end 193.98 66.98) (width 0.25) (layer "B.Cu") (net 20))
 (segment (start 183.82 61.9) (end 186.36 64.44) (width 0.25) (layer "B.Cu") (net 22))
 (segment (start 186.36 64.44) (end 193.98 64.44) (width 0.25) (layer "B.Cu") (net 22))
 (segment (start 146.895 86.125) (end 146.895 80.855) (width 0.25) (layer "F.Cu") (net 34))
 (segment (start 153.34 56.82) (end 145.72 56.82) (width 0.25) (layer "F.Cu") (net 34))
 (segment (start 146.895 80.855) (end 145.72 79.68) (width 0.25) (layer "F.Cu") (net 34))
 (segment (start 186.36 56.82) (end 160.96 56.82) (width 0.25) (layer "F.Cu") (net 34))
 (segment (start 138.1 97.46) (end 145.72 89.84) (width 0.25) (layer "F.Cu") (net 34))
 (segment (start 193.98 49.2) (end 186.36 56.82) (width 0.25) (layer "F.Cu") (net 34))
 (segment (start 140.64 56.82) (end 133.02 56.82) (width 0.25) (layer "F.Cu") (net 34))
 (segment (start 145.72 87.3) (end 146.895 86.125) (width 0.25) (layer "F.Cu") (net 34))
 (segment (start 160.96 56.82) (end 153.34 56.82) (width 0.25) (layer "F.Cu") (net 34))
 (segment (start 125.4 56.82) (end 117.78 56.82) (width 0.25) (layer "F.Cu") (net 34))
 (segment (start 145.72 89.84) (end 145.72 87.3) (width 0.25) (layer "F.Cu") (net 34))
 (segment (start 133.02 56.82) (end 125.4 56.82) (width 0.25) (layer "F.Cu") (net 34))
 (segment (start 145.72 56.82) (end 140.64 56.82) (width 0.25) (layer "F.Cu") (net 34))
 (segment (start 150.8 89.84) (end 150.8 97.46) (width 0.25) (layer "B.Cu") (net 40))
 (segment (start 145.72 84.76) (end 150.8 89.84) (width 0.25) (layer "B.Cu") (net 40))
 (segment (start 152.115 83.535) (end 152.115 96.235) (width 0.25) (layer "B.Cu") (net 41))
 (segment (start 145.72 77.14) (end 152.115 83.535) (width 0.25) (layer "B.Cu") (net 41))
 (segment (start 152.115 96.235) (end 153.34 97.46) (width 0.25) (layer "B.Cu") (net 41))
 (segment (start 135.401 50.375) (end 136.576 49.2) (width 0.25) (layer "B.Cu") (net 62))
 (segment (start 126.765 50.375) (end 135.401 50.375) (width 0.25) (layer "B.Cu") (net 62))
 (segment (start 117.78 59.36) (end 126.765 50.375) (width 0.25) (layer "B.Cu") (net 62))
 (segment (start 138.237701 49.2) (end 139.116 49.2) (width 0.25) (layer "B.Cu") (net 63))
 (segment (start 128.077701 59.36) (end 138.237701 49.2) (width 0.25) (layer "B.Cu") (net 63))
 (segment (start 125.4 59.36) (end 128.077701 59.36) (width 0.25) (layer "B.Cu") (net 63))
 (segment (start 141.656 50.724) (end 141.656 49.2) (width 0.25) (layer "B.Cu") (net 64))
 (segment (start 133.02 59.36) (end 141.656 50.724) (width 0.25) (layer "B.Cu") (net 64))
 (segment (start 145.72 59.36) (end 145.72 58.635) (width 0.25) (layer "F.Cu") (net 65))
 (segment (start 144.545 58.185) (end 144.545 50.375) (width 0.25) (layer "B.Cu") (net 65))
 (segment (start 144.545 50.375) (end 145.72 49.2) (width 0.25) (layer "B.Cu") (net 65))
 (segment (start 145.72 59.36) (end 144.545 58.185) (width 0.25) (layer "B.Cu") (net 65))
 (segment (start 148.26 54.28) (end 148.26 49.2) (width 0.25) (layer "B.Cu") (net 66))
 (segment (start 153.34 59.36) (end 148.26 54.28) (width 0.25) (layer "B.Cu") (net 66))
 (segment (start 152.615 51.015) (end 150.8 49.2) (width 0.25) (layer "B.Cu") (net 67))
 (segment (start 152.615 53.555) (end 152.615 51.015) (width 0.25) (layer "B.Cu") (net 67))
 (segment (start 158.42 59.36) (end 160.96 59.36) (width 0.25) (layer "B.Cu") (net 67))
 (segment (start 158.42 59.36) (end 152.615 53.555) (width 0.25) (layer "B.Cu") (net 67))
 (segment (start 115.24 59.36) (end 115.24 54.28) (width 0.25) (layer "F.Cu") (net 69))
 (segment (start 154.705 50.375) (end 155.88 49.2) (width 0.25) (layer "F.Cu") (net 69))
 (segment (start 115.24 54.28) (end 117.78 51.74) (width 0.25) (layer "F.Cu") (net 69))
 (segment (start 147.085 50.375) (end 154.705 50.375) (width 0.25) (layer "F.Cu") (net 69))
 (segment (start 117.78 61.9) (end 115.24 59.36) (width 0.25) (layer "F.Cu") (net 69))
 (segment (start 117.78 61.9) (end 125.4 61.9) (width 0.25) (layer "F.Cu") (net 69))
 (segment (start 125.4 61.9) (end 133.02 61.9) (width 0.25) (layer "F.Cu") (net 69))
 (segment (start 145.72 51.74) (end 147.085 50.375) (width 0.25) (layer "F.Cu") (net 69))
 (segment (start 117.78 51.74) (end 145.72 51.74) (width 0.25) (layer "F.Cu") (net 69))
 (segment (start 163.5 54.28) (end 158.42 49.2) (width 0.25) (layer "B.Cu") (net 70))
 (segment (start 153.34 61.9) (end 160.96 61.9) (width 0.25) (layer "B.Cu") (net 70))
 (segment (start 145.72 61.9) (end 153.34 61.9) (width 0.25) (layer "B.Cu") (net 70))
 (segment (start 160.96 61.9) (end 163.5 59.36) (width 0.25) (layer "B.Cu") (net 70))
 (segment (start 163.5 59.36) (end 163.5 54.28) (width 0.25) (layer "B.Cu") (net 70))
 (segment (start 155.88 89.84) (end 163.5 82.22) (width 2) (layer "F.Cu") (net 79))
 (segment (start 148.26 69.52) (end 131.9 69.52) (width 2) (layer "F.Cu") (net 79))
 (segment (start 155.88 77.14) (end 148.26 69.52) (width 2) (layer "F.Cu") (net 79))
 (segment (start 155.88 89.84) (end 155.88 77.14) (width 2) (layer "F.Cu") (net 79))
 (segment (start 131.9 69.52) (end 126.82 74.6) (width 2) (layer "F.Cu") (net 79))
 (segment (start 163.5 82.22) (end 176.2 82.22) (width 2) (layer "F.Cu") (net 79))
 (segment (start 181.28 92.38) (end 181.28 82.22) (width 1) (layer "F.Cu") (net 39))
 (segment (start 148.26 94.92) (end 178.74 94.92) (width 1) (layer "F.Cu") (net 39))
 (segment (start 145.72 97.46) (end 148.26 94.92) (width 1) (layer "F.Cu") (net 39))
 (segment (start 178.74 94.92) (end 181.28 92.38) (width 1) (layer "F.Cu") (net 39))
 (segment (start 115.24 87.3) (end 117.78 89.84) (width 2) (layer "F.Cu") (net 80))
 (segment (start 115.24 77.14) (end 115.24 87.3) (width 2) (layer "F.Cu") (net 80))
 (segment (start 117.78 89.84) (end 130.48 89.84) (width 2) (layer "F.Cu") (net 80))
 (segment (start 117.78 74.6) (end 115.24 77.14) (width 2) (layer "F.Cu") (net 80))
 (segment (start 122.86 74.6) (end 117.78 74.6) (width 2) (layer "F.Cu") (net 80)))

